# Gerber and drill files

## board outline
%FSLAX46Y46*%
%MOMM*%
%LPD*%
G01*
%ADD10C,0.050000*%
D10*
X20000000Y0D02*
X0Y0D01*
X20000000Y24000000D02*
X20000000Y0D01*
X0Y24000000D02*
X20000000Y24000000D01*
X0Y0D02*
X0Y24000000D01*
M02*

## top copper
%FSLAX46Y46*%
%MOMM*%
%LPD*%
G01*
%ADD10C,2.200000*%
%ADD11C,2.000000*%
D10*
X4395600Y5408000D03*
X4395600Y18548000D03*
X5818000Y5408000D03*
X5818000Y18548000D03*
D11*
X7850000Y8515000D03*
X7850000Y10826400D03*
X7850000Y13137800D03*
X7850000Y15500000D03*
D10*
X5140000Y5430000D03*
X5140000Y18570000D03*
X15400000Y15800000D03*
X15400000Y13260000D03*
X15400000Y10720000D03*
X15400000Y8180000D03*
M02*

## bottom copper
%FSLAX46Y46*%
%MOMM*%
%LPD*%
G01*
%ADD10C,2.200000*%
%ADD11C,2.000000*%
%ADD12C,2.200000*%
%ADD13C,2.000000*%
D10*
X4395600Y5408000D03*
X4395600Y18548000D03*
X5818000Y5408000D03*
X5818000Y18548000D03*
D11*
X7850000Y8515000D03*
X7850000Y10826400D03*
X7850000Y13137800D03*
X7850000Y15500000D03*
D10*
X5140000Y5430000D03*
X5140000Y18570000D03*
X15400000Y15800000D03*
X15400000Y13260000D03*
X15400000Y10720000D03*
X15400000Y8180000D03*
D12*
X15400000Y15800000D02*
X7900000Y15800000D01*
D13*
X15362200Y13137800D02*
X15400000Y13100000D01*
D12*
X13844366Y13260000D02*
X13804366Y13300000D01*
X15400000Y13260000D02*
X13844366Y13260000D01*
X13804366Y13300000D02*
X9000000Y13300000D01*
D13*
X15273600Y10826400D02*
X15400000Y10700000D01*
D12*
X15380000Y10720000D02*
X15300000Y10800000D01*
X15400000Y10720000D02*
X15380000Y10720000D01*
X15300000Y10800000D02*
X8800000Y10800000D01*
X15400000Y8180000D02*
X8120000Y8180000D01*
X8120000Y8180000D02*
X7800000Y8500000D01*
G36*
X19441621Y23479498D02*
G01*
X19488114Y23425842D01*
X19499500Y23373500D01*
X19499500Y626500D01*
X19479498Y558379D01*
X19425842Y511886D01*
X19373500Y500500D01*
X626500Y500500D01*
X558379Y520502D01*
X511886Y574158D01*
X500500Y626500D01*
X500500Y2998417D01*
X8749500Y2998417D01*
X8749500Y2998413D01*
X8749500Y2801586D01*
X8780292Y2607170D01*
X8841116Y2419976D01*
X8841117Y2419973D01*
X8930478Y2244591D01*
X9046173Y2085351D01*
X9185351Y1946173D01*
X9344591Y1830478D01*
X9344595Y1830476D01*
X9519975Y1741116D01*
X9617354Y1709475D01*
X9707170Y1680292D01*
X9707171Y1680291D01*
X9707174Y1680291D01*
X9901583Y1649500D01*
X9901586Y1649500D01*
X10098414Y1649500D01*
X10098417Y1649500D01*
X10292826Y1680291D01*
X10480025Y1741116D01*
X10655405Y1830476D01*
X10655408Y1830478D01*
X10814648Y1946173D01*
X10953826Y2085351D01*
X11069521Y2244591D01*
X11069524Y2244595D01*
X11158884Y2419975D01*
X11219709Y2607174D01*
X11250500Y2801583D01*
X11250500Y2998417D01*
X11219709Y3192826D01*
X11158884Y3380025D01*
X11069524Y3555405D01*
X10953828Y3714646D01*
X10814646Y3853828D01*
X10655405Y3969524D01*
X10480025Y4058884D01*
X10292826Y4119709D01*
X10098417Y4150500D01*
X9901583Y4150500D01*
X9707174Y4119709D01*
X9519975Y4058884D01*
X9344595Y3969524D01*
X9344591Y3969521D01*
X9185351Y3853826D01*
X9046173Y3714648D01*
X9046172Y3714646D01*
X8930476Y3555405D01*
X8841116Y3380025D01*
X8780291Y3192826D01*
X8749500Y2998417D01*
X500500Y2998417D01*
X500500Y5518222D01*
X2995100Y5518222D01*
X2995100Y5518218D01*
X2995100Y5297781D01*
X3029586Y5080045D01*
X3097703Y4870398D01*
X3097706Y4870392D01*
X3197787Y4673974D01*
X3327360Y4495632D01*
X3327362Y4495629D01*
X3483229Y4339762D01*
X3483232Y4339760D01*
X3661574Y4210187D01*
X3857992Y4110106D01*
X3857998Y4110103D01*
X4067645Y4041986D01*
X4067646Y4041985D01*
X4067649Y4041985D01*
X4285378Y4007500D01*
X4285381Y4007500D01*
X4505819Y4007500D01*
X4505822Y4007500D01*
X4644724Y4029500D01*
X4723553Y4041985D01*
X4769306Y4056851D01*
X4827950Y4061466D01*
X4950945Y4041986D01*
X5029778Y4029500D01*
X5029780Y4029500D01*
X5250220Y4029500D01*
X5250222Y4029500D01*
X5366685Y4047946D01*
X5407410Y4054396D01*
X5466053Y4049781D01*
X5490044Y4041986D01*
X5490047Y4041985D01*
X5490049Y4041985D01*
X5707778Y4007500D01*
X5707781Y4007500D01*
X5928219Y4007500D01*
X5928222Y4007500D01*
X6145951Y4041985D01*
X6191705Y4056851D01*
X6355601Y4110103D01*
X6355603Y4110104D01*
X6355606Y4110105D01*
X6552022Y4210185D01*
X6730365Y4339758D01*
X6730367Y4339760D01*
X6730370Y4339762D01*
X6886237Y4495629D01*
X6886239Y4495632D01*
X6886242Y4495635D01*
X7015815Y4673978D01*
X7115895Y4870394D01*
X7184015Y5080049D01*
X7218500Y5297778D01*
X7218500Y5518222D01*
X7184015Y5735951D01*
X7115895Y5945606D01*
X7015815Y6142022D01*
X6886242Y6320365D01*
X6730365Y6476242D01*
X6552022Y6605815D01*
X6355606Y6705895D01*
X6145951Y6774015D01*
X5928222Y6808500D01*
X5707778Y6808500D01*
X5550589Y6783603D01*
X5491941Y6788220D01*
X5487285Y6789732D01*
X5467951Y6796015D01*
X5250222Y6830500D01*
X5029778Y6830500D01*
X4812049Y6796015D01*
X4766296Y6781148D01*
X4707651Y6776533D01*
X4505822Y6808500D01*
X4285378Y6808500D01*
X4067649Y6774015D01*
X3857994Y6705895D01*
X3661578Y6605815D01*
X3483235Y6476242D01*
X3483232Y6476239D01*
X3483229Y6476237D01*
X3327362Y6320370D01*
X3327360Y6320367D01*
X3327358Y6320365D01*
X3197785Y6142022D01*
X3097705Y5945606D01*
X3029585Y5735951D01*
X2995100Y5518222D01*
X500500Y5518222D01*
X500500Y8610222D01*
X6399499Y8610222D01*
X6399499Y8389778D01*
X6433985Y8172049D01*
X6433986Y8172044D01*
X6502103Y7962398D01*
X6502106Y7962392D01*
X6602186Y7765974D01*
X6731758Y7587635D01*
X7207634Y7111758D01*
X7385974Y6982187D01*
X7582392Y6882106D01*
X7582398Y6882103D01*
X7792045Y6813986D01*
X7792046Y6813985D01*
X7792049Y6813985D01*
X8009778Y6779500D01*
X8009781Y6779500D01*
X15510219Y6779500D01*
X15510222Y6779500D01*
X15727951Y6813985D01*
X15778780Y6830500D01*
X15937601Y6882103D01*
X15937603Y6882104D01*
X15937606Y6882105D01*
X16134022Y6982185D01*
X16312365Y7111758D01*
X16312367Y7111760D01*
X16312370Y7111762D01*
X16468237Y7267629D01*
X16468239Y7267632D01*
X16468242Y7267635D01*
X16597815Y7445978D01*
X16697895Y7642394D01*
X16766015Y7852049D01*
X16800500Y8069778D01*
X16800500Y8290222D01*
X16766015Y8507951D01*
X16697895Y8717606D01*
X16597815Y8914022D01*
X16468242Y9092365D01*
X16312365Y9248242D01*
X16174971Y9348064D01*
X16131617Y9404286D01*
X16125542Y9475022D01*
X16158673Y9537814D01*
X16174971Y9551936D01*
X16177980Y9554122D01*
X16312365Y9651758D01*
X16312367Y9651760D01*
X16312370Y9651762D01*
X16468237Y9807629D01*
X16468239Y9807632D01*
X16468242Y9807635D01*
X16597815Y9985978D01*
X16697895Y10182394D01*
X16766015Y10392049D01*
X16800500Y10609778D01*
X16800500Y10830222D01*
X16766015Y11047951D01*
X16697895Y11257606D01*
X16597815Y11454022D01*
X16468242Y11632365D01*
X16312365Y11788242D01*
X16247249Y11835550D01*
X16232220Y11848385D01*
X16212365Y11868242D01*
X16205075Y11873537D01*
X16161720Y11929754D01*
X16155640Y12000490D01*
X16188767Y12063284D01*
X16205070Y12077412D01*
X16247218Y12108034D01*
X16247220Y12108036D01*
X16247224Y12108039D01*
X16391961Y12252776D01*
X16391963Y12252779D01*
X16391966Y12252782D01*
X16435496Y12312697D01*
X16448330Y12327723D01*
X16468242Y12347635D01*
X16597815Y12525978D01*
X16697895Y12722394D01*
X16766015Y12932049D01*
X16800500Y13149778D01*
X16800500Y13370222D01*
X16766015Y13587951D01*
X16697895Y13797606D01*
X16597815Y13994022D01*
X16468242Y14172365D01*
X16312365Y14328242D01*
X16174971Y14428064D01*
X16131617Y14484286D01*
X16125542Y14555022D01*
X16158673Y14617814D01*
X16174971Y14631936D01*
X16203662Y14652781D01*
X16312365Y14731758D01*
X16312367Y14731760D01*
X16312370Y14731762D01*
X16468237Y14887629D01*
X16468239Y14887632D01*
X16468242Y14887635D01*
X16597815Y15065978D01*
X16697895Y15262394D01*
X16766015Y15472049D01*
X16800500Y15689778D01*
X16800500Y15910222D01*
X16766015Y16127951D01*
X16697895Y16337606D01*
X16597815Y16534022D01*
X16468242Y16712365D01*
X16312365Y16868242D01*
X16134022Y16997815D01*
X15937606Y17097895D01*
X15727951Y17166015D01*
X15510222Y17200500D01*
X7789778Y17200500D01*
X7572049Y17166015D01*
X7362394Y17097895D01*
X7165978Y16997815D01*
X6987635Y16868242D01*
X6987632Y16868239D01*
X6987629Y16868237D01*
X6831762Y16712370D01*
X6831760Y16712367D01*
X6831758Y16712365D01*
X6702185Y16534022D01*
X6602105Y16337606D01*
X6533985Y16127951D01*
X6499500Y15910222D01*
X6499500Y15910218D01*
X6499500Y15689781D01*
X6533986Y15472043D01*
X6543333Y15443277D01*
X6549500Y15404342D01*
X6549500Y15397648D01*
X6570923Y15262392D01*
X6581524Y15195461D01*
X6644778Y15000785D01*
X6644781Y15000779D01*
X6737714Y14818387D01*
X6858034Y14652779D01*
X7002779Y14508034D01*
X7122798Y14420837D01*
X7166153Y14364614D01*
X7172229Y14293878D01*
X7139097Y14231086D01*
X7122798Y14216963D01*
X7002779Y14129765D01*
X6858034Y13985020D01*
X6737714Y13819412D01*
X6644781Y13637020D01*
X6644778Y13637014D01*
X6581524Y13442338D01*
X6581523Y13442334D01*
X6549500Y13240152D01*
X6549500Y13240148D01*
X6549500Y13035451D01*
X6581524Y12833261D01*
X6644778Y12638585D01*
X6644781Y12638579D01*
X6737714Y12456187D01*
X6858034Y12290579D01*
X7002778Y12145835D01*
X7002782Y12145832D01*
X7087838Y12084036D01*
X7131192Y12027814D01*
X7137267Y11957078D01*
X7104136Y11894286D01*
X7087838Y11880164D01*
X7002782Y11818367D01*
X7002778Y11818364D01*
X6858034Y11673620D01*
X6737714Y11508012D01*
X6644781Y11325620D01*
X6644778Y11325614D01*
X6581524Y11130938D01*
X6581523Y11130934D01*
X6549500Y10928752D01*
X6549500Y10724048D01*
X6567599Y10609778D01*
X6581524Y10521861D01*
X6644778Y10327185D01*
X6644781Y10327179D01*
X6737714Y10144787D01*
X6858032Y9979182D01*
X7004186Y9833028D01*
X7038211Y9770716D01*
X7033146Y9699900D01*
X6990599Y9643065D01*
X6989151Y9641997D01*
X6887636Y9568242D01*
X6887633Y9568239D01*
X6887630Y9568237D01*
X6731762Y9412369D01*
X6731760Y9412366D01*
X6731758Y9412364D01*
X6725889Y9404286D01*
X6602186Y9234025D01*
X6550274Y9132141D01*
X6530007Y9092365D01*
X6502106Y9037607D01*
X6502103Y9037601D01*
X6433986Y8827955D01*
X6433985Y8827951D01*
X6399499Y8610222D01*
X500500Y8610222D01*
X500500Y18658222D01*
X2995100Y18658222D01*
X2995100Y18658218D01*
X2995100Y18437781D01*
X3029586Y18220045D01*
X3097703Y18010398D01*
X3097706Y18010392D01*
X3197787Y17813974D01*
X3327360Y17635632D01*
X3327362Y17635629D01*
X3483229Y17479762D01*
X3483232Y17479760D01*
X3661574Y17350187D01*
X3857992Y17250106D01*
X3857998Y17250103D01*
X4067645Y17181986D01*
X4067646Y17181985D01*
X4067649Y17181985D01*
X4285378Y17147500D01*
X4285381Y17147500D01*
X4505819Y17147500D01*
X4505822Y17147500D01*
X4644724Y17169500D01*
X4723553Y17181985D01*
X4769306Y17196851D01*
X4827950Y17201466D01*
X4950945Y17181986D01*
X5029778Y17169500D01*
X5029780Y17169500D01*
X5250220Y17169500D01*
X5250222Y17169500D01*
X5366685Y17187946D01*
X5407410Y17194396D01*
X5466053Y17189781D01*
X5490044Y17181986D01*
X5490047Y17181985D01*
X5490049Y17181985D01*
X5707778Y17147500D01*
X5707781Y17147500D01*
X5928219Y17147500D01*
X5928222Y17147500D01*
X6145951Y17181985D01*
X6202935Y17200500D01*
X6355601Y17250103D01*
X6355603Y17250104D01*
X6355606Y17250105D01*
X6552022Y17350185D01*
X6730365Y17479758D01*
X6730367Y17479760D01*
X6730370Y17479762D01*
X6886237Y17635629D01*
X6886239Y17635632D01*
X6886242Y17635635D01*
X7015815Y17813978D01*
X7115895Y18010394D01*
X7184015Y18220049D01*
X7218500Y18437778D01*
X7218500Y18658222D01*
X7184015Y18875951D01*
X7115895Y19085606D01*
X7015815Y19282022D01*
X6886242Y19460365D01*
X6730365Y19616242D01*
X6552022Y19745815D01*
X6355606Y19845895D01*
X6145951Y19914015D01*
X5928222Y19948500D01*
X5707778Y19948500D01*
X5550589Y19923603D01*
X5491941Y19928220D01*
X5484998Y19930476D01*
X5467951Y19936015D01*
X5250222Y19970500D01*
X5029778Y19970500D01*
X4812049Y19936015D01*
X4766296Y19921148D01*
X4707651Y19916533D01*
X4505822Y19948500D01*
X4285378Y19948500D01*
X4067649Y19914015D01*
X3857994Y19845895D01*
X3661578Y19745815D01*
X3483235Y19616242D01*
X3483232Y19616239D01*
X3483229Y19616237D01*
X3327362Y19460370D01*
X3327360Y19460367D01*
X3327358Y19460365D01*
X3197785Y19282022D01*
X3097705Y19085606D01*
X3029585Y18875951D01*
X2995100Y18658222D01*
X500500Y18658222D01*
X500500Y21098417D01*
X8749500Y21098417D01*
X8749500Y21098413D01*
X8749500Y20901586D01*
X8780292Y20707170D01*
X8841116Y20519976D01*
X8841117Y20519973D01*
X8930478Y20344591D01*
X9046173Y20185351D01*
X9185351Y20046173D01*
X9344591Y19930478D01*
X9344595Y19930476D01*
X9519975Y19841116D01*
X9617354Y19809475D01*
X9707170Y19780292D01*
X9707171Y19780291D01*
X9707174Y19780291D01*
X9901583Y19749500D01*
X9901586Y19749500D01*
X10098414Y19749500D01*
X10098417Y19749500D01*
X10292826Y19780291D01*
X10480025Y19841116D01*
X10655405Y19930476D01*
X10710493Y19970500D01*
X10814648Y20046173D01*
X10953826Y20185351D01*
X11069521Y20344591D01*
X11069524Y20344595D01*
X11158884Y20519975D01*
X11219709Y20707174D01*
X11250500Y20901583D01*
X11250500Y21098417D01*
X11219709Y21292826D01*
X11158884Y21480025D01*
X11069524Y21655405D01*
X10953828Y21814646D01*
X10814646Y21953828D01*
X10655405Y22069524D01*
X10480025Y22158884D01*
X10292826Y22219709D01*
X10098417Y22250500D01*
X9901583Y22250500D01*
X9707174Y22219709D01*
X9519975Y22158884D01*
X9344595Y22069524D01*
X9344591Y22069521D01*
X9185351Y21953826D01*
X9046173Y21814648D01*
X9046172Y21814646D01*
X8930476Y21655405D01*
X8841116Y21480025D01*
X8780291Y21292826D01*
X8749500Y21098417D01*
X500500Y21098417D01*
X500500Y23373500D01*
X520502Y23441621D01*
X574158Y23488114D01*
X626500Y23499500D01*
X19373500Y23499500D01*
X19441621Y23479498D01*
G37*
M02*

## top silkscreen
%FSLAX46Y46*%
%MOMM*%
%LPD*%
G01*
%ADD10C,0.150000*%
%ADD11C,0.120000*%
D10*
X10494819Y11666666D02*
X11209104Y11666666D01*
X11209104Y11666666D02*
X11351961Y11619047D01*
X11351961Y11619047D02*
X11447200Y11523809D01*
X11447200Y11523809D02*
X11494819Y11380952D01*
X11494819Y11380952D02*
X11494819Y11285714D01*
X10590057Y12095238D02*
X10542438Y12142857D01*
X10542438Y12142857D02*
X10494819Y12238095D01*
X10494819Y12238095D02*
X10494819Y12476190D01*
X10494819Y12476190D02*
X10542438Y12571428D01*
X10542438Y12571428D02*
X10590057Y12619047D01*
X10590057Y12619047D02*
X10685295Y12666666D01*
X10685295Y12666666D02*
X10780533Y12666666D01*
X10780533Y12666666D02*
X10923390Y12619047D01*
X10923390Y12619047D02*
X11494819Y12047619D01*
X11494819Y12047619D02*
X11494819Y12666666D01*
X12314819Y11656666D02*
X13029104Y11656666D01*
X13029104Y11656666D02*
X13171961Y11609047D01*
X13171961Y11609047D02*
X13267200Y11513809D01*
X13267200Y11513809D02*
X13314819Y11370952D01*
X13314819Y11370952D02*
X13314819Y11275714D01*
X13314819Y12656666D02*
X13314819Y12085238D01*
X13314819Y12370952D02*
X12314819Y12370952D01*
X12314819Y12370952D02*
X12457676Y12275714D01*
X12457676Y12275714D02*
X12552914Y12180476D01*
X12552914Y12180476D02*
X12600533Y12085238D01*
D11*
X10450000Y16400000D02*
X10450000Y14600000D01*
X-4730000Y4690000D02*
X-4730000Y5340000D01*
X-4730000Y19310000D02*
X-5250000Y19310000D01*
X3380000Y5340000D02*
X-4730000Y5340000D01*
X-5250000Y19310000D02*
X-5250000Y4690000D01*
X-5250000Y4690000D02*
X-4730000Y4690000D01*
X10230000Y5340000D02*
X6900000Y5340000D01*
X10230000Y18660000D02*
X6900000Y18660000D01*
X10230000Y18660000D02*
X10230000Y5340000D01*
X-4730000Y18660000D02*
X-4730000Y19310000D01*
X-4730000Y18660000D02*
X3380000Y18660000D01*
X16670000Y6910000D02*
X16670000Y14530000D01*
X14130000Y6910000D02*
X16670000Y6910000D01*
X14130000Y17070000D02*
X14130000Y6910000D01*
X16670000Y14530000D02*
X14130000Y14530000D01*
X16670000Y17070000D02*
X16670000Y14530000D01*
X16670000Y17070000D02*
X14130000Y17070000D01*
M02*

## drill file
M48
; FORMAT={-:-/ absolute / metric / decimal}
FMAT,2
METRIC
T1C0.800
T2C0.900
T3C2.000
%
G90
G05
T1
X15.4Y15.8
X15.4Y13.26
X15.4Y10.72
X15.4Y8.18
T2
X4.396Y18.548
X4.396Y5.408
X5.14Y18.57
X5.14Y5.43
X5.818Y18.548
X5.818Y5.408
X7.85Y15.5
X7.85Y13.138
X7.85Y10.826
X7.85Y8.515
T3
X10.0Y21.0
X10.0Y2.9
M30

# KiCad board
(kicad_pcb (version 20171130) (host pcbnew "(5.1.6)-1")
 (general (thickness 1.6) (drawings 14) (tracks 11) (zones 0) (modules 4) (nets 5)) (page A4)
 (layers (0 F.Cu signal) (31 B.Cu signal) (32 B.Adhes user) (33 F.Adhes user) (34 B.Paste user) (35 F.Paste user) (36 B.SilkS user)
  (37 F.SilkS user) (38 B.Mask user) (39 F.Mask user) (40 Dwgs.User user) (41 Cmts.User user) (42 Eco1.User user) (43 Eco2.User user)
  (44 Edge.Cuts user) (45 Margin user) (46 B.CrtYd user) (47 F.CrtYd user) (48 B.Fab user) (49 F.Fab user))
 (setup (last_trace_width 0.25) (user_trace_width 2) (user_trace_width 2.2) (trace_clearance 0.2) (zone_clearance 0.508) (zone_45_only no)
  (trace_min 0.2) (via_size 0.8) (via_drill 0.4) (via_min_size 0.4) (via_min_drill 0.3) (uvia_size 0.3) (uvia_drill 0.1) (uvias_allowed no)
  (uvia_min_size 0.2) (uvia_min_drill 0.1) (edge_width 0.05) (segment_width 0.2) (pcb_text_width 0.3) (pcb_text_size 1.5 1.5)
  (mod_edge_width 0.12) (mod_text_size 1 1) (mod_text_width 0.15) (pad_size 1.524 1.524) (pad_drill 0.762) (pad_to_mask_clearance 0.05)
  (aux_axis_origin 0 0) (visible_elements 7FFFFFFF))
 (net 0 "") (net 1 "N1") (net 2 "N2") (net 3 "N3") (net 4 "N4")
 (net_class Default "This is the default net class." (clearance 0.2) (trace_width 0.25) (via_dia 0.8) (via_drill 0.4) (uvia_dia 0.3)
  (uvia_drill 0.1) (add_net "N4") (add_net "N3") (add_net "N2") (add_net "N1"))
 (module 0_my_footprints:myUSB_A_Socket (layer F.Cu) (at 7.85 -15.5 270)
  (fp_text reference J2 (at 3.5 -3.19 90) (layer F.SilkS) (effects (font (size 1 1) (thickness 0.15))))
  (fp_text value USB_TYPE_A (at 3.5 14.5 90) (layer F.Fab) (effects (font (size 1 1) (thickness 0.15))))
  (fp_line (start -0.9 -2.6) (end 0.9 -2.6) (layer F.SilkS) (width 0.12))
  (fp_line (start 10.81 12.58) (end 10.16 12.58) (layer F.SilkS) (width 0.12))
  (fp_line (start -3.81 12.58) (end -3.81 13.1) (layer F.SilkS) (width 0.12))
  (fp_line (start 10.16 4.47) (end 10.16 12.58) (layer F.SilkS) (width 0.12))
  (fp_line (start -3.81 13.1) (end 10.81 13.1) (layer F.SilkS) (width 0.12))
  (fp_line (start 10.81 13.1) (end 10.81 12.58) (layer F.SilkS) (width 0.12))
  (fp_line (start 10.16 -2.38) (end 10.16 0.95) (layer F.SilkS) (width 0.12))
  (fp_line (start -3.16 -2.38) (end -3.16 0.95) (layer F.SilkS) (width 0.12))
  (fp_line (start -3.16 -2.38) (end 10.16 -2.38) (layer F.SilkS) (width 0.12))
  (fp_line (start -3.16 12.58) (end -3.81 12.58) (layer F.SilkS) (width 0.12))
  (fp_line (start -3.16 12.58) (end -3.16 4.47) (layer F.SilkS) (width 0.12))
  (pad "" thru_hole circle (at 10.092 3.4544 270) (size 2.2 2.2) (drill 0.9) (layers *.Cu *.Mask))
  (pad "" thru_hole circle (at -3.048 3.4544 270) (size 2.2 2.2) (drill 0.9) (layers *.Cu *.Mask))
  (pad "" thru_hole circle (at 10.092 2.032 270) (size 2.2 2.2) (drill 0.9) (layers *.Cu *.Mask))
  (pad "" thru_hole circle (at -3.048 2.032 270) (size 2.2 2.2) (drill 0.9) (layers *.Cu *.Mask))
  (pad 4 thru_hole circle (at 6.985 0 270) (size 2 2) (drill 0.9) (layers *.Cu *.Mask) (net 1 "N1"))
  (pad 3 thru_hole circle (at 4.6736 0 270) (size 2 2) (drill 0.9) (layers *.Cu *.Mask) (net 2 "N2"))
  (pad 2 thru_hole circle (at 2.3622 0 270) (size 2 2) (drill 0.9) (layers *.Cu *.Mask) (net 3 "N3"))
  (pad 1 thru_hole circle (at 0 0 270) (size 2 2) (drill 0.9) (layers *.Cu *.Mask) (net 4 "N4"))
  (pad "" thru_hole circle (at 10.07 2.71 270) (size 2.2 2.2) (drill 0.9) (layers *.Cu *.Mask))
  (pad "" thru_hole circle (at -3.07 2.71 270) (size 2.2 2.2) (drill 0.9) (layers *.Cu *.Mask)))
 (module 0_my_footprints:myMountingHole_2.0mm (layer F.Cu) (at 10 -2.9)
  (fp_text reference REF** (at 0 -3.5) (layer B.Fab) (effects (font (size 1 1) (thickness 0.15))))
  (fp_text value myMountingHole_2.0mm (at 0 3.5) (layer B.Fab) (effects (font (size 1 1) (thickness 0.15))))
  (pad "" np_thru_hole circle (at 0 0) (size 2 2) (drill 2) (layers *.Cu *.Mask)))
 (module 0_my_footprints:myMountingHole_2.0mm (layer F.Cu) (at 10 -21)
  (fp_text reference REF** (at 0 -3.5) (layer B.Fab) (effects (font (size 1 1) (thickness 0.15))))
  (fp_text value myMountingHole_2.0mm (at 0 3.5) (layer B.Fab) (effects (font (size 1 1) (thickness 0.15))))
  (pad "" np_thru_hole circle (at 0 0) (size 2 2) (drill 2) (layers *.Cu *.Mask)))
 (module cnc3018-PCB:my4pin (layer F.Cu) (at 15.4 -15.8 270)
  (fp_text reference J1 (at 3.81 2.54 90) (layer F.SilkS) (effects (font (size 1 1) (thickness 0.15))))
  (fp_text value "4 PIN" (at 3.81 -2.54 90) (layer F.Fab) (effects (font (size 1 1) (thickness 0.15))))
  (fp_line (start 8.89 -1.27) (end 1.27 -1.27) (layer F.SilkS) (width 0.12))
  (fp_line (start 8.89 1.27) (end 8.89 -1.27) (layer F.SilkS) (width 0.12))
  (fp_line (start -1.27 1.27) (end 8.89 1.27) (layer F.SilkS) (width 0.12))
  (fp_line (start 1.27 -1.27) (end 1.27 1.27) (layer F.SilkS) (width 0.12))
  (fp_line (start -1.27 -1.27) (end 1.27 -1.27) (layer F.SilkS) (width 0.12))
  (fp_line (start -1.27 -1.27) (end -1.27 1.27) (layer F.SilkS) (width 0.12))
  (pad 1 thru_hole circle (at 0 0 270) (size 2.2 2.2) (drill 0.8) (layers *.Cu *.Mask) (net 4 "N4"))
  (pad 2 thru_hole circle (at 2.54 0 270) (size 2.2 2.2) (drill 0.8) (layers *.Cu *.Mask) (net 3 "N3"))
  (pad 3 thru_hole circle (at 5.08 0 270) (size 2.2 2.2) (drill 0.8) (layers *.Cu *.Mask) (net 2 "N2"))
  (pad 4 thru_hole circle (at 7.62 0 270) (size 2.2 2.2) (drill 0.8) (layers *.Cu *.Mask) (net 1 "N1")))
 (gr_line (start 20 0) (end 0 0) (layer Edge.Cuts) (width 0.05))
 (gr_line (start 20 -24) (end 20 0) (layer Edge.Cuts) (width 0.05))
 (gr_line (start 0 -24) (end 20 -24) (layer Edge.Cuts) (width 0.05))
 (gr_line (start 0 0) (end 0 -24) (layer Edge.Cuts) (width 0.05))
 (segment (start 15.4 -15.8) (end 7.9 -15.8) (width 2.2) (layer B.Cu) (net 4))
 (segment (start 15.3622 -13.1378) (end 15.4 -13.1) (width 2) (layer B.Cu) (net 3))
 (segment (start 13.844366 -13.26) (end 13.804366 -13.3) (width 2.2) (layer B.Cu) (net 3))
 (segment (start 15.4 -13.26) (end 13.844366 -13.26) (width 2.2) (layer B.Cu) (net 3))
 (segment (start 13.804366 -13.3) (end 9 -13.3) (width 2.2) (layer B.Cu) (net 3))
 (segment (start 15.2736 -10.8264) (end 15.4 -10.7) (width 2) (layer B.Cu) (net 2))
 (segment (start 15.38 -10.72) (end 15.3 -10.8) (width 2.2) (layer B.Cu) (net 2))
 (segment (start 15.4 -10.72) (end 15.38 -10.72) (width 2.2) (layer B.Cu) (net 2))
 (segment (start 15.3 -10.8) (end 8.8 -10.8) (width 2.2) (layer B.Cu) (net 2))
 (segment (start 15.4 -8.18) (end 8.12 -8.18) (width 2.2) (layer B.Cu) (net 1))
 (segment (start 8.12 -8.18) (end 7.8 -8.5) (width 2.2) (layer B.Cu) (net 1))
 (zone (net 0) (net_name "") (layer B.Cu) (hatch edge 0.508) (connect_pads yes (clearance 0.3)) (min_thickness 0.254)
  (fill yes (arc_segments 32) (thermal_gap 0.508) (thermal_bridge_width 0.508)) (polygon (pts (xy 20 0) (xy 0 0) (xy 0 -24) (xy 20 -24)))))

